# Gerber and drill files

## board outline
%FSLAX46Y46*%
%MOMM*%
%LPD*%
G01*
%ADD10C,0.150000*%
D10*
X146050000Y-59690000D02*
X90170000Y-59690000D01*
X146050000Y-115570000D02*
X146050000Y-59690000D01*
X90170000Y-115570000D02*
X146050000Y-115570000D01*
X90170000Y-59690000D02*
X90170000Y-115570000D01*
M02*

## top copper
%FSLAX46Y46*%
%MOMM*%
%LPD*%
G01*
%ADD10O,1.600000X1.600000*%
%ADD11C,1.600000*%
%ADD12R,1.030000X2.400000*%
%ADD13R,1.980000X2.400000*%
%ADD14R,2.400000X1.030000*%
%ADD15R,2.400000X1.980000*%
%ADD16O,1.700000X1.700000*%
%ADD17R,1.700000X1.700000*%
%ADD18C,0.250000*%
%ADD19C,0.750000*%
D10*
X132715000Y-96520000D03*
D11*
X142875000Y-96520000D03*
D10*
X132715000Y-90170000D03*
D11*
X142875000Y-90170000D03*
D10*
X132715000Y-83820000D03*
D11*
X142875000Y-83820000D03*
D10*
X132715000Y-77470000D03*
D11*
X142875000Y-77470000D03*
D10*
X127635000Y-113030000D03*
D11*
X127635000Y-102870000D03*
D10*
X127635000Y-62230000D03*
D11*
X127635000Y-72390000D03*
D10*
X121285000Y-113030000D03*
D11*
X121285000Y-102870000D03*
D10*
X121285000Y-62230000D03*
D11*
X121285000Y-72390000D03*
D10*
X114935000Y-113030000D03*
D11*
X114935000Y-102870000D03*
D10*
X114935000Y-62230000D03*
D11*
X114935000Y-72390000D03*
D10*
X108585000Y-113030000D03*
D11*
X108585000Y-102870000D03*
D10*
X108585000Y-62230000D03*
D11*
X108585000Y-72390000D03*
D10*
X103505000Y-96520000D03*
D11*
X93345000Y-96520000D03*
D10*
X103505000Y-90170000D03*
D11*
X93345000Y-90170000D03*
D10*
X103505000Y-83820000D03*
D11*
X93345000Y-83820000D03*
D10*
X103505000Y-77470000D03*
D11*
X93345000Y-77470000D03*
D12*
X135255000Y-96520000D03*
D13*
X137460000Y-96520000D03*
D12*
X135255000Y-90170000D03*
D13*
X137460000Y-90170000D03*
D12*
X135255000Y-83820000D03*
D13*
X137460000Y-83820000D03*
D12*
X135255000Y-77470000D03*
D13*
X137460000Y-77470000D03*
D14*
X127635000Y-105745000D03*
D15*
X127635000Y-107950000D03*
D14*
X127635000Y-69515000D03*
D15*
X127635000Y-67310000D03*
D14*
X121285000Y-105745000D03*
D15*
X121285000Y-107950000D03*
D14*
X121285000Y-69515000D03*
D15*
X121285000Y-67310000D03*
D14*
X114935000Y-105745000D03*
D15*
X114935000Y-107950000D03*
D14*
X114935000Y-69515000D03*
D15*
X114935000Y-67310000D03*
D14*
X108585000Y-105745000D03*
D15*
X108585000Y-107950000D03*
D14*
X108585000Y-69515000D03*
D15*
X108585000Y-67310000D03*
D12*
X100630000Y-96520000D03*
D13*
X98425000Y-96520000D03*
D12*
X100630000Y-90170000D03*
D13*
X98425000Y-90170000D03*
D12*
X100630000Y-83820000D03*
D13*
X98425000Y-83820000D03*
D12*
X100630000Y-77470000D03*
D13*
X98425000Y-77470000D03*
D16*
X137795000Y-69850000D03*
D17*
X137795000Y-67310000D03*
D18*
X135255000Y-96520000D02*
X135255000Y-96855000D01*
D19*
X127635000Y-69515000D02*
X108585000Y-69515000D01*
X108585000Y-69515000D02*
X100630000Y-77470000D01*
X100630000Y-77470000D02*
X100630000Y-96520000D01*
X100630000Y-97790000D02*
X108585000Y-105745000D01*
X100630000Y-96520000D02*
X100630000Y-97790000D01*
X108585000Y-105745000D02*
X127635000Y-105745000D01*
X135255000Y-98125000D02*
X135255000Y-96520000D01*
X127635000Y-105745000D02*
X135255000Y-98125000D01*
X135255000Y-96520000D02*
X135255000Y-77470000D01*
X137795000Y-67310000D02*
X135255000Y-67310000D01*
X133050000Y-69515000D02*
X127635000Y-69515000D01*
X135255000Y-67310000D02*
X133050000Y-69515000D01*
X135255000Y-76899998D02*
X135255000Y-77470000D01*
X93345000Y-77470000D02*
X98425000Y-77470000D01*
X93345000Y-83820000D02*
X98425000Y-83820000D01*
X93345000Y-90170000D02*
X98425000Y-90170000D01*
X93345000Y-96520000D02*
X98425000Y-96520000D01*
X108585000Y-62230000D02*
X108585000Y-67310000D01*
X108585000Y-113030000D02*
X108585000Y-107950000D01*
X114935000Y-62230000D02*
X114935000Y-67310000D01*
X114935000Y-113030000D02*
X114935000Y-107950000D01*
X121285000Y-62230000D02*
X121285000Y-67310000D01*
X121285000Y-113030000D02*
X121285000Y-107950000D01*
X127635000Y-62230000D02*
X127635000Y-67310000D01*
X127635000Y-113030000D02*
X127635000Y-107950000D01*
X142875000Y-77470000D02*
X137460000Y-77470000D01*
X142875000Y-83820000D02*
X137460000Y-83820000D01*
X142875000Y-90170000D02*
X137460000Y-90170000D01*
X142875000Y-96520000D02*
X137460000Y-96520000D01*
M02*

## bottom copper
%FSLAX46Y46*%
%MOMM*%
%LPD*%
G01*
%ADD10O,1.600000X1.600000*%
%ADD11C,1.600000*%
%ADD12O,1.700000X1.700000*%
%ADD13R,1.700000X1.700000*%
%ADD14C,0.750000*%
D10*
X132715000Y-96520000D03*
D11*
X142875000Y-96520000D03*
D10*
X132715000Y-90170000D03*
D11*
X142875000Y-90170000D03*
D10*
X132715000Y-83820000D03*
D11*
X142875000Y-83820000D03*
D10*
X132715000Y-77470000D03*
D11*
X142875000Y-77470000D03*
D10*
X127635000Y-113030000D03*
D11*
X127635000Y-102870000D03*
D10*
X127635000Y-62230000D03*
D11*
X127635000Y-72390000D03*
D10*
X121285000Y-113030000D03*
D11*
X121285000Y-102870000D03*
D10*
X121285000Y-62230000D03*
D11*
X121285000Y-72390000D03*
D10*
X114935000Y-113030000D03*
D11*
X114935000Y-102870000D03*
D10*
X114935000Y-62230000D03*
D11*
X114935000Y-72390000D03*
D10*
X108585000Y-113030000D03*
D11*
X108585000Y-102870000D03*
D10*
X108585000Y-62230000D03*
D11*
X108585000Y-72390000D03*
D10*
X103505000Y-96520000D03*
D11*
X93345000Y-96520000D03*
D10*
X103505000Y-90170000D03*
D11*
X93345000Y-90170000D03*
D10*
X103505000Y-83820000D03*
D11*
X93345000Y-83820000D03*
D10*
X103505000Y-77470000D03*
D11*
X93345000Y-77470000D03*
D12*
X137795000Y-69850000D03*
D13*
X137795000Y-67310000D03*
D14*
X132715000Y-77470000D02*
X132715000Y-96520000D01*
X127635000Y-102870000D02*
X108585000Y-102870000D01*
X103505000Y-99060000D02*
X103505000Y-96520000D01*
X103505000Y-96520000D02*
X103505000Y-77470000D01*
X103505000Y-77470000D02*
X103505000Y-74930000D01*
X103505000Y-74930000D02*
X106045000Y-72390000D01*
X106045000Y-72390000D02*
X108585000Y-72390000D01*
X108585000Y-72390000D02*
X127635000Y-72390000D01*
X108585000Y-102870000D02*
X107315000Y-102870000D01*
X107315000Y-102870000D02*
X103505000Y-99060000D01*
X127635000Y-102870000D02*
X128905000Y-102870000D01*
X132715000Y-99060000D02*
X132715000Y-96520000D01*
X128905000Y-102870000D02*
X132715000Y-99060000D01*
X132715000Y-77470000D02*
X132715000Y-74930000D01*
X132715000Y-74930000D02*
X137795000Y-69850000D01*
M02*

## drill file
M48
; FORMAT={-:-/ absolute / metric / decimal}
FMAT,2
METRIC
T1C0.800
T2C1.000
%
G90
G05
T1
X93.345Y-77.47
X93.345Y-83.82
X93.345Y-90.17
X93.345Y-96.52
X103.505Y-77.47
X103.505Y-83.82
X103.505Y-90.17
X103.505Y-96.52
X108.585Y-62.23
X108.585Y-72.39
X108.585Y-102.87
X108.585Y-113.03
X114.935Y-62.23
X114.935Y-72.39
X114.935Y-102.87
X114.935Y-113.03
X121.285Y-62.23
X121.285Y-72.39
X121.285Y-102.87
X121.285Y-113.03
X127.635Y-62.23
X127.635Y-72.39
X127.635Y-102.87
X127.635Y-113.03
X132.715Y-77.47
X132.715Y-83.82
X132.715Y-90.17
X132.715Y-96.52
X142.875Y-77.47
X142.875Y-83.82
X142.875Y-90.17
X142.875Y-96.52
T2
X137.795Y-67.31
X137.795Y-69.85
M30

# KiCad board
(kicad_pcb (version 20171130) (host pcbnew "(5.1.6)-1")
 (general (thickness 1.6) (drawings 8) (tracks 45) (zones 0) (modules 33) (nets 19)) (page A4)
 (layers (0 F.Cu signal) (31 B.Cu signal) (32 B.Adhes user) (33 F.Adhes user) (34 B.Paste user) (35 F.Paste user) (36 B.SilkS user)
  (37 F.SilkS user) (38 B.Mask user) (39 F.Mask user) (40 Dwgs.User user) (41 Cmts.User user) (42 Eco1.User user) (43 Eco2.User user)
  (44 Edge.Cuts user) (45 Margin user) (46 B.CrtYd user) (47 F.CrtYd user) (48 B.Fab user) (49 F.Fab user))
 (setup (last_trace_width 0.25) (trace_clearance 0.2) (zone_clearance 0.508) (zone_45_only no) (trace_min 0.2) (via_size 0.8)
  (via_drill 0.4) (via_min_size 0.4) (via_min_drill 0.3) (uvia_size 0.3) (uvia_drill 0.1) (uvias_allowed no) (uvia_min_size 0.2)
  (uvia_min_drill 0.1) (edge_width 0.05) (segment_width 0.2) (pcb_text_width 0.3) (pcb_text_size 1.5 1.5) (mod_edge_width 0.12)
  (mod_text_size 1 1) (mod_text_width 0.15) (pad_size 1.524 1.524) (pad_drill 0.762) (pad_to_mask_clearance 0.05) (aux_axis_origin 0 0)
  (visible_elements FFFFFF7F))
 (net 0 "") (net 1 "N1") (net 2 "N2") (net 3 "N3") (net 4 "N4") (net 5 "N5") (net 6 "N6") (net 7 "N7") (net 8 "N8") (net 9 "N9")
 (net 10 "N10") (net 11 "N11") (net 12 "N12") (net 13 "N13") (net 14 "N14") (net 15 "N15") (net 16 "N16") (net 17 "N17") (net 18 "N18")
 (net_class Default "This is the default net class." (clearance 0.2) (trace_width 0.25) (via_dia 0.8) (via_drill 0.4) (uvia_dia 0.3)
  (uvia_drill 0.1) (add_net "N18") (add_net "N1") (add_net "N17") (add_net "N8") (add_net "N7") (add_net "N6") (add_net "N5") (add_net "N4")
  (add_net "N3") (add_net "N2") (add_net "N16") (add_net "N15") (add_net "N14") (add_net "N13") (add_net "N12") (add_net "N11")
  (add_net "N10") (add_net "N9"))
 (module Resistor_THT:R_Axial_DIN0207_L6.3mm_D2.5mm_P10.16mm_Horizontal (layer B.Cu) (at 142.875 96.52 180)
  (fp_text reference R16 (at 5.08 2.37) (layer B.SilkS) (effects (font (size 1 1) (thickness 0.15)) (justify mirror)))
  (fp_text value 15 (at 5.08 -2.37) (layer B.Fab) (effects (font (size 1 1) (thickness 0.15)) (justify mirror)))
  (pad 2 thru_hole oval (at 10.16 0 180) (size 1.6 1.6) (drill 0.8) (layers *.Cu *.Mask) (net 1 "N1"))
  (pad 1 thru_hole circle (at 0 0 180) (size 1.6 1.6) (drill 0.8) (layers *.Cu *.Mask) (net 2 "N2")))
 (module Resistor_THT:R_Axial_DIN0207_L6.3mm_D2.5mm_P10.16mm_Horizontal (layer B.Cu) (at 142.875 90.17 180)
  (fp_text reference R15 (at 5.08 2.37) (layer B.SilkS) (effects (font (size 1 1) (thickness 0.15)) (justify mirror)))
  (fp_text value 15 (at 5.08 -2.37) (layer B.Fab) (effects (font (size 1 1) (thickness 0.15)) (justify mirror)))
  (pad 2 thru_hole oval (at 10.16 0 180) (size 1.6 1.6) (drill 0.8) (layers *.Cu *.Mask) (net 1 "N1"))
  (pad 1 thru_hole circle (at 0 0 180) (size 1.6 1.6) (drill 0.8) (layers *.Cu *.Mask) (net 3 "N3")))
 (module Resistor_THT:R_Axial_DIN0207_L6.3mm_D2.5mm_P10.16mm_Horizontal (layer B.Cu) (at 142.875 83.82 180)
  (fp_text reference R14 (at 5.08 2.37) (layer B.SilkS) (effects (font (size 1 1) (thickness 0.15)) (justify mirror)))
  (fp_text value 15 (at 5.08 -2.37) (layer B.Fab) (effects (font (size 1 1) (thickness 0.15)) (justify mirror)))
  (pad 2 thru_hole oval (at 10.16 0 180) (size 1.6 1.6) (drill 0.8) (layers *.Cu *.Mask) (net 1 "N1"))
  (pad 1 thru_hole circle (at 0 0 180) (size 1.6 1.6) (drill 0.8) (layers *.Cu *.Mask) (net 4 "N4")))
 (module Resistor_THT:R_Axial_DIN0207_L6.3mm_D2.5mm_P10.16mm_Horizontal (layer B.Cu) (at 142.875 77.47 180)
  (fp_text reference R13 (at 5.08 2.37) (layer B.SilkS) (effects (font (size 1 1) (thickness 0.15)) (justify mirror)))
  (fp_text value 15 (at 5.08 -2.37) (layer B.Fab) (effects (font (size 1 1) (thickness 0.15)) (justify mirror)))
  (pad 2 thru_hole oval (at 10.16 0 180) (size 1.6 1.6) (drill 0.8) (layers *.Cu *.Mask) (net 1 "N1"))
  (pad 1 thru_hole circle (at 0 0 180) (size 1.6 1.6) (drill 0.8) (layers *.Cu *.Mask) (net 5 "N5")))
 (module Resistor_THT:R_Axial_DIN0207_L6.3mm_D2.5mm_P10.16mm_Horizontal (layer B.Cu) (at 127.635 102.87 270)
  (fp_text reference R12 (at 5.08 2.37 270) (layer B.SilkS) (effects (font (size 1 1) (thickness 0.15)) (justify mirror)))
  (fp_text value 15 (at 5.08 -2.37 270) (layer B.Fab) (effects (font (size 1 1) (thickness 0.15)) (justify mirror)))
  (pad 2 thru_hole oval (at 10.16 0 270) (size 1.6 1.6) (drill 0.8) (layers *.Cu *.Mask) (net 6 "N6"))
  (pad 1 thru_hole circle (at 0 0 270) (size 1.6 1.6) (drill 0.8) (layers *.Cu *.Mask) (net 1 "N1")))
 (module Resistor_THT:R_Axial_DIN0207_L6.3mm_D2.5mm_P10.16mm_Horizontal (layer B.Cu) (at 127.635 72.39 90)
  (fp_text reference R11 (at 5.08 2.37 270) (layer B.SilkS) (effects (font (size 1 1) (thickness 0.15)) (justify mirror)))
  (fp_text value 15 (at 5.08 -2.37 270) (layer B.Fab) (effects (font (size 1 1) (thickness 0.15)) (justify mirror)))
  (pad 2 thru_hole oval (at 10.16 0 90) (size 1.6 1.6) (drill 0.8) (layers *.Cu *.Mask) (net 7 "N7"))
  (pad 1 thru_hole circle (at 0 0 90) (size 1.6 1.6) (drill 0.8) (layers *.Cu *.Mask) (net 1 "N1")))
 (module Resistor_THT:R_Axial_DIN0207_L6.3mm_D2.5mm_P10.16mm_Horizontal (layer B.Cu) (at 121.285 102.87 270)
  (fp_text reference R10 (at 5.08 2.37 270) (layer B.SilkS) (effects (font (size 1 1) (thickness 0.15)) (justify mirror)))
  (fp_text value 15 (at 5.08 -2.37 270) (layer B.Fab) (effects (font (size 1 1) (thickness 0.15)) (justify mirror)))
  (pad 2 thru_hole oval (at 10.16 0 270) (size 1.6 1.6) (drill 0.8) (layers *.Cu *.Mask) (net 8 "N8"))
  (pad 1 thru_hole circle (at 0 0 270) (size 1.6 1.6) (drill 0.8) (layers *.Cu *.Mask) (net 1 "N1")))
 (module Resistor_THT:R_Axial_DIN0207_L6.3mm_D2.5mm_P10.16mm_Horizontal (layer B.Cu) (at 121.285 72.39 90)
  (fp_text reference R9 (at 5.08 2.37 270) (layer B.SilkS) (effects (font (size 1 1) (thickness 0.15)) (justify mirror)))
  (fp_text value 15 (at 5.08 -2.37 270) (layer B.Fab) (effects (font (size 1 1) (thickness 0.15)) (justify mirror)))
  (pad 2 thru_hole oval (at 10.16 0 90) (size 1.6 1.6) (drill 0.8) (layers *.Cu *.Mask) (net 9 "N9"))
  (pad 1 thru_hole circle (at 0 0 90) (size 1.6 1.6) (drill 0.8) (layers *.Cu *.Mask) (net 1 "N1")))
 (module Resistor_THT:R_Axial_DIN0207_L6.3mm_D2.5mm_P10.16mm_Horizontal (layer B.Cu) (at 114.935 102.87 270)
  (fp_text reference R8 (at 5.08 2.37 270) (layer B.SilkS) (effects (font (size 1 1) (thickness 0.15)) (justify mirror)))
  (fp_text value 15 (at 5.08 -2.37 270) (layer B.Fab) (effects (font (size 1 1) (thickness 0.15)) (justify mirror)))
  (pad 2 thru_hole oval (at 10.16 0 270) (size 1.6 1.6) (drill 0.8) (layers *.Cu *.Mask) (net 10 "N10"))
  (pad 1 thru_hole circle (at 0 0 270) (size 1.6 1.6) (drill 0.8) (layers *.Cu *.Mask) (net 1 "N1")))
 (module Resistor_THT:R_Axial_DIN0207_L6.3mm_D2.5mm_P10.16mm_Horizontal (layer B.Cu) (at 114.935 72.39 90)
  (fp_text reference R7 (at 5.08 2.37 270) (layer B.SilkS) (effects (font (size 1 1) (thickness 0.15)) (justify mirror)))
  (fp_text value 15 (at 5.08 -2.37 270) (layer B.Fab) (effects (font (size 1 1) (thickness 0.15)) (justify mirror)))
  (pad 2 thru_hole oval (at 10.16 0 90) (size 1.6 1.6) (drill 0.8) (layers *.Cu *.Mask) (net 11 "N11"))
  (pad 1 thru_hole circle (at 0 0 90) (size 1.6 1.6) (drill 0.8) (layers *.Cu *.Mask) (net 1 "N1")))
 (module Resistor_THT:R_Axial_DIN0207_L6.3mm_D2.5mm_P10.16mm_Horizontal (layer B.Cu) (at 108.585 102.87 270)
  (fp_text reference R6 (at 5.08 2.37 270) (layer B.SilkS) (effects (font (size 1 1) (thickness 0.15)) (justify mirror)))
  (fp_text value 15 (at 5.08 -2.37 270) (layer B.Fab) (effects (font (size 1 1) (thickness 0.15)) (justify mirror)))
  (pad 2 thru_hole oval (at 10.16 0 270) (size 1.6 1.6) (drill 0.8) (layers *.Cu *.Mask) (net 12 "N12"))
  (pad 1 thru_hole circle (at 0 0 270) (size 1.6 1.6) (drill 0.8) (layers *.Cu *.Mask) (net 1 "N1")))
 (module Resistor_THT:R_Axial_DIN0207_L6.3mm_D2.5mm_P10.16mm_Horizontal (layer B.Cu) (at 108.585 72.39 90)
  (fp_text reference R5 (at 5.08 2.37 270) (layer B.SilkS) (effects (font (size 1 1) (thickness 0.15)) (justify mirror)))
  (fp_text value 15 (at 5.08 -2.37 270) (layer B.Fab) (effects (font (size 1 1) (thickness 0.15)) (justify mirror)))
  (pad 2 thru_hole oval (at 10.16 0 90) (size 1.6 1.6) (drill 0.8) (layers *.Cu *.Mask) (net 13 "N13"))
  (pad 1 thru_hole circle (at 0 0 90) (size 1.6 1.6) (drill 0.8) (layers *.Cu *.Mask) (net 1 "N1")))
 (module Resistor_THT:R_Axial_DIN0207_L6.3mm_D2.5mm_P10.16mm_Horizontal (layer B.Cu) (at 93.345 96.52)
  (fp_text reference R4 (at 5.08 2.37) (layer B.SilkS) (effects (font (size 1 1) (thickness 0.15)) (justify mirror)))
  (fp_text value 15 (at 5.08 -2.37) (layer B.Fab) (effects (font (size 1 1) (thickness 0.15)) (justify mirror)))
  (pad 2 thru_hole oval (at 10.16 0) (size 1.6 1.6) (drill 0.8) (layers *.Cu *.Mask) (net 1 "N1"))
  (pad 1 thru_hole circle (at 0 0) (size 1.6 1.6) (drill 0.8) (layers *.Cu *.Mask) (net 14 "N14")))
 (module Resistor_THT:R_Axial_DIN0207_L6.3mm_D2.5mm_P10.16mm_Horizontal (layer B.Cu) (at 93.345 90.17)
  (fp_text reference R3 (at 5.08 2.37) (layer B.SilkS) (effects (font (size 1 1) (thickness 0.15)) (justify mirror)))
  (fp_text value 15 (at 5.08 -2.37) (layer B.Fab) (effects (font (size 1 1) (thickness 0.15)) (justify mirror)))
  (pad 2 thru_hole oval (at 10.16 0) (size 1.6 1.6) (drill 0.8) (layers *.Cu *.Mask) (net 1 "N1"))
  (pad 1 thru_hole circle (at 0 0) (size 1.6 1.6) (drill 0.8) (layers *.Cu *.Mask) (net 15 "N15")))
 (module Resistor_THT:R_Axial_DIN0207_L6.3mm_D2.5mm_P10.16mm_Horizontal (layer B.Cu) (at 93.345 83.82)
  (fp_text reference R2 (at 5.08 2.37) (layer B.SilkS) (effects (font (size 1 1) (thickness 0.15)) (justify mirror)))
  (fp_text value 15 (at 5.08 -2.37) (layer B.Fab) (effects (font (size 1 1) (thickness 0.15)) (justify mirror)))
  (pad 2 thru_hole oval (at 10.16 0) (size 1.6 1.6) (drill 0.8) (layers *.Cu *.Mask) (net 1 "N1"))
  (pad 1 thru_hole circle (at 0 0) (size 1.6 1.6) (drill 0.8) (layers *.Cu *.Mask) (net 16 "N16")))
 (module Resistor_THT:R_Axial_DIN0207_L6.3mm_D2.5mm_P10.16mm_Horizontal (layer B.Cu) (at 93.345 77.47)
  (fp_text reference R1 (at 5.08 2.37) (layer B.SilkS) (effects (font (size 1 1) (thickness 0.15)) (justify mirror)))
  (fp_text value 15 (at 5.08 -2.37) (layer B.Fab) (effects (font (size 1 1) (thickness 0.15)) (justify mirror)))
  (pad 2 thru_hole oval (at 10.16 0) (size 1.6 1.6) (drill 0.8) (layers *.Cu *.Mask) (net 1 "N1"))
  (pad 1 thru_hole circle (at 0 0) (size 1.6 1.6) (drill 0.8) (layers *.Cu *.Mask) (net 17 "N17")))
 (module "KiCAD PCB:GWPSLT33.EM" (layer F.Cu) (at 136.6 96.52 180)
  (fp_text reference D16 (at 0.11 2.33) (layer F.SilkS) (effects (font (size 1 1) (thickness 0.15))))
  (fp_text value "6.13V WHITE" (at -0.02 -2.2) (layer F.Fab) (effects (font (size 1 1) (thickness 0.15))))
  (pad 2 smd rect (at 1.345 0 180) (size 1.03 2.4) (layers F.Cu F.Paste F.Mask) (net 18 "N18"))
  (pad 1 smd rect (at -0.86 0 180) (size 1.98 2.4) (layers F.Cu F.Paste F.Mask) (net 2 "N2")))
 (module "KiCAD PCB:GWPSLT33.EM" (layer F.Cu) (at 136.6 90.17 180)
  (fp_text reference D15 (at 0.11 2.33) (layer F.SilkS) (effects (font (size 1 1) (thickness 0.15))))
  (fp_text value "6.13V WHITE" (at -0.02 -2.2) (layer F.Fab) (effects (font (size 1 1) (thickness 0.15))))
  (pad 2 smd rect (at 1.345 0 180) (size 1.03 2.4) (layers F.Cu F.Paste F.Mask) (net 18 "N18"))
  (pad 1 smd rect (at -0.86 0 180) (size 1.98 2.4) (layers F.Cu F.Paste F.Mask) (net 3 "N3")))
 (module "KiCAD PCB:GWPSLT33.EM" (layer F.Cu) (at 136.6 83.82 180)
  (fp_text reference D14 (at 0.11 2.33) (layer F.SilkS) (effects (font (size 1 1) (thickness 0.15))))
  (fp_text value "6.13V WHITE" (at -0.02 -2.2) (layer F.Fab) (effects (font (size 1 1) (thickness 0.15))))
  (pad 2 smd rect (at 1.345 0 180) (size 1.03 2.4) (layers F.Cu F.Paste F.Mask) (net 18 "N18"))
  (pad 1 smd rect (at -0.86 0 180) (size 1.98 2.4) (layers F.Cu F.Paste F.Mask) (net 4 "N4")))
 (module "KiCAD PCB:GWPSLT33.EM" (layer F.Cu) (at 136.6 77.47 180)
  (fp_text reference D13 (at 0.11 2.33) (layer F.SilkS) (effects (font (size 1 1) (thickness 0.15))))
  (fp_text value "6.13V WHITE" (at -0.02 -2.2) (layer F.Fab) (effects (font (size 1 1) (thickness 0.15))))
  (pad 2 smd rect (at 1.345 0 180) (size 1.03 2.4) (layers F.Cu F.Paste F.Mask) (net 18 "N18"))
  (pad 1 smd rect (at -0.86 0 180) (size 1.98 2.4) (layers F.Cu F.Paste F.Mask) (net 5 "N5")))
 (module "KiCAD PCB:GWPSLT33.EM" (layer F.Cu) (at 127.635 107.09 90)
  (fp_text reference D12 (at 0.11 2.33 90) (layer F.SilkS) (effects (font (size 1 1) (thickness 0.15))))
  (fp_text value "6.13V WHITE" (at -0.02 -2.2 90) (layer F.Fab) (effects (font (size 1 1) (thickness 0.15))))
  (pad 2 smd rect (at 1.345 0 90) (size 1.03 2.4) (layers F.Cu F.Paste F.Mask) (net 18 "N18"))
  (pad 1 smd rect (at -0.86 0 90) (size 1.98 2.4) (layers F.Cu F.Paste F.Mask) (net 6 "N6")))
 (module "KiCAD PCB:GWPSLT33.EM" (layer F.Cu) (at 127.635 68.17 270)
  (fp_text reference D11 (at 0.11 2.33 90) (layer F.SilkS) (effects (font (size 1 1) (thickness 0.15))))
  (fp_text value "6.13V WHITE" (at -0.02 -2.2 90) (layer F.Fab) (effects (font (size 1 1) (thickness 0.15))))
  (pad 2 smd rect (at 1.345 0 270) (size 1.03 2.4) (layers F.Cu F.Paste F.Mask) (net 18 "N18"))
  (pad 1 smd rect (at -0.86 0 270) (size 1.98 2.4) (layers F.Cu F.Paste F.Mask) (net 7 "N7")))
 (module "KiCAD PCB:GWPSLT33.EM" (layer F.Cu) (at 121.285 107.09 90)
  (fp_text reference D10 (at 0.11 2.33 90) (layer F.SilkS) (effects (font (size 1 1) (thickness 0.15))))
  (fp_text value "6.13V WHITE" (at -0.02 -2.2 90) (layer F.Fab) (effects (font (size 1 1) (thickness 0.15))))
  (pad 2 smd rect (at 1.345 0 90) (size 1.03 2.4) (layers F.Cu F.Paste F.Mask) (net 18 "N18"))
  (pad 1 smd rect (at -0.86 0 90) (size 1.98 2.4) (layers F.Cu F.Paste F.Mask) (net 8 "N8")))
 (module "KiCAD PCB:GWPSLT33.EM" (layer F.Cu) (at 121.285 68.17 270)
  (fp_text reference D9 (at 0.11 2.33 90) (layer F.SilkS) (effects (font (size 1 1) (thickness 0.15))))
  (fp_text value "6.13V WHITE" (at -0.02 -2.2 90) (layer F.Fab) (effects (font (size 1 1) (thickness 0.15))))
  (pad 2 smd rect (at 1.345 0 270) (size 1.03 2.4) (layers F.Cu F.Paste F.Mask) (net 18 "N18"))
  (pad 1 smd rect (at -0.86 0 270) (size 1.98 2.4) (layers F.Cu F.Paste F.Mask) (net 9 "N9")))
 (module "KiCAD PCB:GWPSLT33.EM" (layer F.Cu) (at 114.935 107.09 90)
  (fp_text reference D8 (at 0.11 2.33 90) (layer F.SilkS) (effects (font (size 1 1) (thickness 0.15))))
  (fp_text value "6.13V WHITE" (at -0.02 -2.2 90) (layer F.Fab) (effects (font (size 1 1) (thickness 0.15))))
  (pad 2 smd rect (at 1.345 0 90) (size 1.03 2.4) (layers F.Cu F.Paste F.Mask) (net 18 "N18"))
  (pad 1 smd rect (at -0.86 0 90) (size 1.98 2.4) (layers F.Cu F.Paste F.Mask) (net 10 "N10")))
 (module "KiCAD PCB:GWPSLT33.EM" (layer F.Cu) (at 114.935 68.17 270)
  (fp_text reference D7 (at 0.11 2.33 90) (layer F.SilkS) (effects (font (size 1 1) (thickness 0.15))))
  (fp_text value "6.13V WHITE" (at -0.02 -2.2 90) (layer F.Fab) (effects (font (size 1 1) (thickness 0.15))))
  (pad 2 smd rect (at 1.345 0 270) (size 1.03 2.4) (layers F.Cu F.Paste F.Mask) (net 18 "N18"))
  (pad 1 smd rect (at -0.86 0 270) (size 1.98 2.4) (layers F.Cu F.Paste F.Mask) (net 11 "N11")))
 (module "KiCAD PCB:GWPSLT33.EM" (layer F.Cu) (at 108.585 107.09 90)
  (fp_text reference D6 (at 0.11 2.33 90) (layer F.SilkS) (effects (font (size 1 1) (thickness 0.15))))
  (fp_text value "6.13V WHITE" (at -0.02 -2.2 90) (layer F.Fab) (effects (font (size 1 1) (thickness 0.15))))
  (pad 2 smd rect (at 1.345 0 90) (size 1.03 2.4) (layers F.Cu F.Paste F.Mask) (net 18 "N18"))
  (pad 1 smd rect (at -0.86 0 90) (size 1.98 2.4) (layers F.Cu F.Paste F.Mask) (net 12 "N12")))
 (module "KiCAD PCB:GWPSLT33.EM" (layer F.Cu) (at 108.585 68.17 270)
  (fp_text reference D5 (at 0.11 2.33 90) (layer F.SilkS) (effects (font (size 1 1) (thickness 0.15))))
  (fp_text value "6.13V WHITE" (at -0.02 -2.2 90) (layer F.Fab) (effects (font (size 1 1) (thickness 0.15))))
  (pad 2 smd rect (at 1.345 0 270) (size 1.03 2.4) (layers F.Cu F.Paste F.Mask) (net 18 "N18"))
  (pad 1 smd rect (at -0.86 0 270) (size 1.98 2.4) (layers F.Cu F.Paste F.Mask) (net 13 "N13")))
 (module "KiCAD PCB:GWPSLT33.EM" (layer F.Cu) (at 99.285 96.52)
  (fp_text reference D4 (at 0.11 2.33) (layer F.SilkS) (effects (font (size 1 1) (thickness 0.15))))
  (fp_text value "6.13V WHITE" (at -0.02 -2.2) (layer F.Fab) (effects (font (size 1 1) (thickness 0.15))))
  (pad 2 smd rect (at 1.345 0) (size 1.03 2.4) (layers F.Cu F.Paste F.Mask) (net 18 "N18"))
  (pad 1 smd rect (at -0.86 0) (size 1.98 2.4) (layers F.Cu F.Paste F.Mask) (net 14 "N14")))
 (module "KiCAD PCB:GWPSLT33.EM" (layer F.Cu) (at 99.285 90.17)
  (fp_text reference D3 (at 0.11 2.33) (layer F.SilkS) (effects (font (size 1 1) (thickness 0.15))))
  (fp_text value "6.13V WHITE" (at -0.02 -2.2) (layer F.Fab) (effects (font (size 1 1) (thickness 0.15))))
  (pad 2 smd rect (at 1.345 0) (size 1.03 2.4) (layers F.Cu F.Paste F.Mask) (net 18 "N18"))
  (pad 1 smd rect (at -0.86 0) (size 1.98 2.4) (layers F.Cu F.Paste F.Mask) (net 15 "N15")))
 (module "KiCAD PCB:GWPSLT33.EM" (layer F.Cu) (at 99.285 83.82)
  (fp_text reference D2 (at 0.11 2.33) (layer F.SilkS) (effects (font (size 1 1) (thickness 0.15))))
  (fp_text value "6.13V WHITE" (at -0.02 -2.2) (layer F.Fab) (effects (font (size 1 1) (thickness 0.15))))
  (pad 2 smd rect (at 1.345 0) (size 1.03 2.4) (layers F.Cu F.Paste F.Mask) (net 18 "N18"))
  (pad 1 smd rect (at -0.86 0) (size 1.98 2.4) (layers F.Cu F.Paste F.Mask) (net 16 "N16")))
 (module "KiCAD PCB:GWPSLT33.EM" (layer F.Cu) (at 99.285 77.47)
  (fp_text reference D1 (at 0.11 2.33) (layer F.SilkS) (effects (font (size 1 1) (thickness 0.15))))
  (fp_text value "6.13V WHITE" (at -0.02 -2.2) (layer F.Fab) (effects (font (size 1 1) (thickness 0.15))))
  (pad 2 smd rect (at 1.345 0) (size 1.03 2.4) (layers F.Cu F.Paste F.Mask) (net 18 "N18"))
  (pad 1 smd rect (at -0.86 0) (size 1.98 2.4) (layers F.Cu F.Paste F.Mask) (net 17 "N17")))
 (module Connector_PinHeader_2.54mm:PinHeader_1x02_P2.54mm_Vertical (layer F.Cu) (at 137.795 67.31)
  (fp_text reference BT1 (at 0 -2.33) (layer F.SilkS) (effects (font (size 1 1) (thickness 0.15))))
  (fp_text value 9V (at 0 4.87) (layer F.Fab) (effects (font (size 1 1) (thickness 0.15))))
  (pad 2 thru_hole oval (at 0 2.54) (size 1.7 1.7) (drill 1) (layers *.Cu *.Mask) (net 1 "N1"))
  (pad 1 thru_hole rect (at 0 0) (size 1.7 1.7) (drill 1) (layers *.Cu *.Mask) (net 18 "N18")))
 (gr_line (start 146.05 59.69) (end 90.17 59.69) (layer Edge.Cuts) (width 0.15))
 (gr_line (start 146.05 115.57) (end 146.05 59.69) (layer Edge.Cuts) (width 0.15))
 (gr_line (start 90.17 115.57) (end 146.05 115.57) (layer Edge.Cuts) (width 0.15))
 (gr_line (start 90.17 59.69) (end 90.17 115.57) (layer Edge.Cuts) (width 0.15))
 (segment (start 132.715 77.47) (end 132.715 96.52) (width 0.75) (layer B.Cu) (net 1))
 (segment (start 127.635 102.87) (end 108.585 102.87) (width 0.75) (layer B.Cu) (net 1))
 (segment (start 103.505 99.06) (end 103.505 96.52) (width 0.75) (layer B.Cu) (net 1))
 (segment (start 103.505 96.52) (end 103.505 77.47) (width 0.75) (layer B.Cu) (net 1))
 (segment (start 103.505 77.47) (end 103.505 74.93) (width 0.75) (layer B.Cu) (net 1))
 (segment (start 103.505 74.93) (end 106.045 72.39) (width 0.75) (layer B.Cu) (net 1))
 (segment (start 106.045 72.39) (end 108.585 72.39) (width 0.75) (layer B.Cu) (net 1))
 (segment (start 108.585 72.39) (end 127.635 72.39) (width 0.75) (layer B.Cu) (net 1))
 (segment (start 108.585 102.87) (end 107.315 102.87) (width 0.75) (layer B.Cu) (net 1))
 (segment (start 107.315 102.87) (end 103.505 99.06) (width 0.75) (layer B.Cu) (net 1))
 (segment (start 127.635 102.87) (end 128.905 102.87) (width 0.75) (layer B.Cu) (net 1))
 (segment (start 132.715 99.06) (end 132.715 96.52) (width 0.75) (layer B.Cu) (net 1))
 (segment (start 128.905 102.87) (end 132.715 99.06) (width 0.75) (layer B.Cu) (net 1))
 (segment (start 132.715 77.47) (end 132.715 74.93) (width 0.75) (layer B.Cu) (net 1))
 (segment (start 132.715 74.93) (end 137.795 69.85) (width 0.75) (layer B.Cu) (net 1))
 (segment (start 135.255 96.52) (end 135.255 96.855) (width 0.25) (layer F.Cu) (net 18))
 (segment (start 127.635 69.515) (end 108.585 69.515) (width 0.75) (layer F.Cu) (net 18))
 (segment (start 108.585 69.515) (end 100.63 77.47) (width 0.75) (layer F.Cu) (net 18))
 (segment (start 100.63 77.47) (end 100.63 96.52) (width 0.75) (layer F.Cu) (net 18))
 (segment (start 100.63 97.79) (end 108.585 105.745) (width 0.75) (layer F.Cu) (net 18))
 (segment (start 100.63 96.52) (end 100.63 97.79) (width 0.75) (layer F.Cu) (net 18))
 (segment (start 108.585 105.745) (end 127.635 105.745) (width 0.75) (layer F.Cu) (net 18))
 (segment (start 135.255 98.125) (end 135.255 96.52) (width 0.75) (layer F.Cu) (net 18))
 (segment (start 127.635 105.745) (end 135.255 98.125) (width 0.75) (layer F.Cu) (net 18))
 (segment (start 135.255 96.52) (end 135.255 77.47) (width 0.75) (layer F.Cu) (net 18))
 (segment (start 137.795 67.31) (end 135.255 67.31) (width 0.75) (layer F.Cu) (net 18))
 (segment (start 133.05 69.515) (end 127.635 69.515) (width 0.75) (layer F.Cu) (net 18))
 (segment (start 135.255 67.31) (end 133.05 69.515) (width 0.75) (layer F.Cu) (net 18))
 (segment (start 135.255 76.899998) (end 135.255 77.47) (width 0.75) (layer F.Cu) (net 18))
 (segment (start 93.345 77.47) (end 98.425 77.47) (width 0.75) (layer F.Cu) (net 17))
 (segment (start 93.345 83.82) (end 98.425 83.82) (width 0.75) (layer F.Cu) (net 16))
 (segment (start 93.345 90.17) (end 98.425 90.17) (width 0.75) (layer F.Cu) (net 15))
 (segment (start 93.345 96.52) (end 98.425 96.52) (width 0.75) (layer F.Cu) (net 14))
 (segment (start 108.585 62.23) (end 108.585 67.31) (width 0.75) (layer F.Cu) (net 13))
 (segment (start 108.585 113.03) (end 108.585 107.95) (width 0.75) (layer F.Cu) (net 12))
 (segment (start 114.935 62.23) (end 114.935 67.31) (width 0.75) (layer F.Cu) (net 11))
 (segment (start 114.935 113.03) (end 114.935 107.95) (width 0.75) (layer F.Cu) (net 10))
 (segment (start 121.285 62.23) (end 121.285 67.31) (width 0.75) (layer F.Cu) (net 9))
 (segment (start 121.285 113.03) (end 121.285 107.95) (width 0.75) (layer F.Cu) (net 8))
 (segment (start 127.635 62.23) (end 127.635 67.31) (width 0.75) (layer F.Cu) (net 7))
 (segment (start 127.635 113.03) (end 127.635 107.95) (width 0.75) (layer F.Cu) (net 6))
 (segment (start 142.875 77.47) (end 137.46 77.47) (width 0.75) (layer F.Cu) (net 5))
 (segment (start 142.875 83.82) (end 137.46 83.82) (width 0.75) (layer F.Cu) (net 4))
 (segment (start 142.875 90.17) (end 137.46 90.17) (width 0.75) (layer F.Cu) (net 3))
 (segment (start 142.875 96.52) (end 137.46 96.52) (width 0.75) (layer F.Cu) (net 2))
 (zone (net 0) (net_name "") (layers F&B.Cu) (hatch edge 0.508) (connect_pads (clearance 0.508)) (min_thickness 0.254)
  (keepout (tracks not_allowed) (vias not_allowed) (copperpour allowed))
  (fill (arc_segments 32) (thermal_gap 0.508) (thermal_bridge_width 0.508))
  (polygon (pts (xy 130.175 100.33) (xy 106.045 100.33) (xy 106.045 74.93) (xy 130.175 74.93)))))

